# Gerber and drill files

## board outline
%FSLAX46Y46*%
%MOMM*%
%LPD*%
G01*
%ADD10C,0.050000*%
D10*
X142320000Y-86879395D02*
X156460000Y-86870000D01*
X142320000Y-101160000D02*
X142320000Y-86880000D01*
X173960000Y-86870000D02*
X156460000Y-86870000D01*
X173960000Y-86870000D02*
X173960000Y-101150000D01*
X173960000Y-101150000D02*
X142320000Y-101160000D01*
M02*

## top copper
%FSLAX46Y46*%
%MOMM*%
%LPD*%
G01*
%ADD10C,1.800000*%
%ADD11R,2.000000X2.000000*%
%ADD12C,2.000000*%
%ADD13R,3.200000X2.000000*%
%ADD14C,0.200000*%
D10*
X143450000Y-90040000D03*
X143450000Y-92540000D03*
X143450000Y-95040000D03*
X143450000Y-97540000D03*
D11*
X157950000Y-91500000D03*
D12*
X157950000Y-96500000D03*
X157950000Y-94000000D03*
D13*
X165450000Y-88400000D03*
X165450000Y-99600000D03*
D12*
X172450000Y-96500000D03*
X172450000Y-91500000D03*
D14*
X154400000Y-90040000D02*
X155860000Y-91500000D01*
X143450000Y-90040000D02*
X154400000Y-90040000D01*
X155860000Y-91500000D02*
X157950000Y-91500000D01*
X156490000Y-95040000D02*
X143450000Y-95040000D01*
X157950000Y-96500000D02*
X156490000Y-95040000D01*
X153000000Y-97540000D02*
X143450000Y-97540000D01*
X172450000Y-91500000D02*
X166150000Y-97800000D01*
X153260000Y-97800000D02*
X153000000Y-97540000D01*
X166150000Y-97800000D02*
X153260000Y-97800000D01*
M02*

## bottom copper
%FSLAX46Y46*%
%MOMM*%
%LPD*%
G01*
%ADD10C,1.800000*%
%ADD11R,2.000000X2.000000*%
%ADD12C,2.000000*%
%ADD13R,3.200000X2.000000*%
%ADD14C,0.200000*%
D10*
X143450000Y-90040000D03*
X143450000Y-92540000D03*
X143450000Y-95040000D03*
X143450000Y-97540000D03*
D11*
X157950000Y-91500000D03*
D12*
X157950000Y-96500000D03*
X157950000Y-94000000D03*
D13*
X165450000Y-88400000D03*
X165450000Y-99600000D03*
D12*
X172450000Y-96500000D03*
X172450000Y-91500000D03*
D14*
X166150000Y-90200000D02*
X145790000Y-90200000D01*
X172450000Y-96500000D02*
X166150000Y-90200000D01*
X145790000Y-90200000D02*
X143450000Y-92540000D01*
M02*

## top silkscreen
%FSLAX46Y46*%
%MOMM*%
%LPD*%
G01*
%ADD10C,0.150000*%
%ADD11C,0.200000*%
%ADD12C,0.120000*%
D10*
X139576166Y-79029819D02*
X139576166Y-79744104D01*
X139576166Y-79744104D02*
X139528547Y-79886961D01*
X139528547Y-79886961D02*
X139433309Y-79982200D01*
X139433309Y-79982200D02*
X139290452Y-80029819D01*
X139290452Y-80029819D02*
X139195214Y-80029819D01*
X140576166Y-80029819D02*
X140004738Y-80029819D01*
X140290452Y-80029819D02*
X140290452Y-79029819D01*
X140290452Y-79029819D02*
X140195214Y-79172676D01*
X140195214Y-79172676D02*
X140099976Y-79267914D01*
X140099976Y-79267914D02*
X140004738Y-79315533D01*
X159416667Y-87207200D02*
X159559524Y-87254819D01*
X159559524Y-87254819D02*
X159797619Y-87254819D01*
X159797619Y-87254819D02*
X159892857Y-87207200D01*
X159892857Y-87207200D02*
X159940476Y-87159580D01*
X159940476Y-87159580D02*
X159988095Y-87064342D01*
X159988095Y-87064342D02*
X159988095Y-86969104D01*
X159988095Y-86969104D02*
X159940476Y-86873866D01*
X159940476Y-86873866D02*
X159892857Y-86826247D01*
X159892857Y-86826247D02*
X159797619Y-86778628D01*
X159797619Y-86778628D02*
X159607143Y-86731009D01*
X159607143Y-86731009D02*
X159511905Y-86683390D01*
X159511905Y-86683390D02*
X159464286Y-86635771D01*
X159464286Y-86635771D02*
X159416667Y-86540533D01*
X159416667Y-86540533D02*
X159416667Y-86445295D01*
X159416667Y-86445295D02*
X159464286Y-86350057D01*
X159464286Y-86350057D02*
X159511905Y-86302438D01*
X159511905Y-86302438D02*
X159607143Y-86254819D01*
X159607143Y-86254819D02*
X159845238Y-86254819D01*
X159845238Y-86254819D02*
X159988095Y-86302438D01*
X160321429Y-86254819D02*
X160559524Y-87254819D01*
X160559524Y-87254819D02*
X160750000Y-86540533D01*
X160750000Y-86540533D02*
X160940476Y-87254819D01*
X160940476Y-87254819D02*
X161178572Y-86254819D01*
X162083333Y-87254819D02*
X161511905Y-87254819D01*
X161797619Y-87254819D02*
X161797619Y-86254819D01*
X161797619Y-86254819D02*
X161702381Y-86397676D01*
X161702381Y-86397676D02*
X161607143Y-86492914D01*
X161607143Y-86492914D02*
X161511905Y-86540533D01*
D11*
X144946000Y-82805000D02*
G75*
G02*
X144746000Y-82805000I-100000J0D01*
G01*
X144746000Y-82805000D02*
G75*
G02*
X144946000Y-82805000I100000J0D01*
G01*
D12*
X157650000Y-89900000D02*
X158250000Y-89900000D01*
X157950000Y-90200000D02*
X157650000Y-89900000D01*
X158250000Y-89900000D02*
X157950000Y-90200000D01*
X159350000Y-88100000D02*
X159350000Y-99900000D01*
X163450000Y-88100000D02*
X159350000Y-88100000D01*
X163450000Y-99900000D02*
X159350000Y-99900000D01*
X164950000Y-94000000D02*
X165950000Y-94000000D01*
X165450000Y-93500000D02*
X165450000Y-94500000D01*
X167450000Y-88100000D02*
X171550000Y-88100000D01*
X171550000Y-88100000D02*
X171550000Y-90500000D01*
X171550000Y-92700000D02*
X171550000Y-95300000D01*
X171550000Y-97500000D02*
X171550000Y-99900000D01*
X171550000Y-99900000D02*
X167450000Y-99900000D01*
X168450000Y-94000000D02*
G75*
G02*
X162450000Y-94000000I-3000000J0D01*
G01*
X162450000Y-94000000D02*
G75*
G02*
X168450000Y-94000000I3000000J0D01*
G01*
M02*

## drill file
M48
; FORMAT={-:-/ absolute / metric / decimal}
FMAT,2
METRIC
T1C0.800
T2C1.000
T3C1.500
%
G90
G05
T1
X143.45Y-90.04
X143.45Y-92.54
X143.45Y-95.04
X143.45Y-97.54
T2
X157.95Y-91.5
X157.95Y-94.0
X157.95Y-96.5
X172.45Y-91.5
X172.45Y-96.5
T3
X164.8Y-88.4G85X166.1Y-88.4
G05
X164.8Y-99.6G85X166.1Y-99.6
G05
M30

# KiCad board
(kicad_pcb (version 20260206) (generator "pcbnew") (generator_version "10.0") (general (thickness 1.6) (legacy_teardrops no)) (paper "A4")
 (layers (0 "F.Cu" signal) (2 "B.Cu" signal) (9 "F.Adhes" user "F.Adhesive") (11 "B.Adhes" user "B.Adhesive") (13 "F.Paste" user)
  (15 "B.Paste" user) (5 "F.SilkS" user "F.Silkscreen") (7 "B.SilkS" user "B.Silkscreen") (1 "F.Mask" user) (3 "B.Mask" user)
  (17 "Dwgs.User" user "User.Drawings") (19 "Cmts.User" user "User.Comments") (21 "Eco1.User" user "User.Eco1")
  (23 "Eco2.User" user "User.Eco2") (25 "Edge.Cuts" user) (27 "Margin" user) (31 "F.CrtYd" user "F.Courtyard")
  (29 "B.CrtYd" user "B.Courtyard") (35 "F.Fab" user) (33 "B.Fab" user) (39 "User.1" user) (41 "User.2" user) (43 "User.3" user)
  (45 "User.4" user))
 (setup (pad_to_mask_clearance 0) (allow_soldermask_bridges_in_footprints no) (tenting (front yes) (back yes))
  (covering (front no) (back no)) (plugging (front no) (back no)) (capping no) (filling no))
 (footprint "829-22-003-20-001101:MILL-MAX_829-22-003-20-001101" (layer "F.Cu") (at 140.25 82.19)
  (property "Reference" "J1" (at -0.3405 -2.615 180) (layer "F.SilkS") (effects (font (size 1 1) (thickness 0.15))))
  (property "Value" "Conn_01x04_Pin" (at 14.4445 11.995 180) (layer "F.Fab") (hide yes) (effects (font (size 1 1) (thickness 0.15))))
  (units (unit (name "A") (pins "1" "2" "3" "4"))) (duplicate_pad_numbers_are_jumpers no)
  (fp_circle (center 4.596 0.615) (end 4.596 0.715) (stroke (width 0.2) (type solid)) (fill no) (layer "F.SilkS"))
  (pad "1" thru_hole circle (at 3.2 7.85 270) (size 1.8 1.8) (drill 0.8) (layers "*.Cu" "*.Mask") (remove_unused_layers no) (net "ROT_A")
   (solder_mask_margin 0.102))
  (pad "2" thru_hole circle (at 3.2 10.35 270) (size 1.8 1.8) (drill 0.8) (layers "*.Cu" "*.Mask") (remove_unused_layers no) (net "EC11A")
   (solder_mask_margin 0.102))
  (pad "3" thru_hole circle (at 3.2 12.85 270) (size 1.8 1.8) (drill 0.8) (layers "*.Cu" "*.Mask") (remove_unused_layers no) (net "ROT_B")
   (solder_mask_margin 0.102))
  (pad "4" thru_hole circle (at 3.2 15.35 270) (size 1.8 1.8) (drill 0.8) (layers "*.Cu" "*.Mask") (remove_unused_layers no) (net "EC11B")
   (solder_mask_margin 0.102)))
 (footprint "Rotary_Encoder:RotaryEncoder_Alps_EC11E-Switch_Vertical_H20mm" (layer "F.Cu") (at 157.95 91.5)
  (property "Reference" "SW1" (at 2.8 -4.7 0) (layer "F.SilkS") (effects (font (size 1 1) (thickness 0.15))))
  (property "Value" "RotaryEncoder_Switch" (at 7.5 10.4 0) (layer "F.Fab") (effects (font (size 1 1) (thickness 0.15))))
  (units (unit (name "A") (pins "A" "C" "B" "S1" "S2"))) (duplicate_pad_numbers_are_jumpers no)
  (fp_line (start -0.3 -1.6) (end 0.3 -1.6) (stroke (width 0.12) (type solid)) (layer "F.SilkS"))
  (fp_line (start 0 -1.3) (end -0.3 -1.6) (stroke (width 0.12) (type solid)) (layer "F.SilkS"))
  (fp_line (start 0.3 -1.6) (end 0 -1.3) (stroke (width 0.12) (type solid)) (layer "F.SilkS"))
  (fp_line (start 1.4 -3.4) (end 1.4 8.4) (stroke (width 0.12) (type solid)) (layer "F.SilkS"))
  (fp_line (start 5.5 -3.4) (end 1.4 -3.4) (stroke (width 0.12) (type solid)) (layer "F.SilkS"))
  (fp_line (start 5.5 8.4) (end 1.4 8.4) (stroke (width 0.12) (type solid)) (layer "F.SilkS"))
  (fp_line (start 7 2.5) (end 8 2.5) (stroke (width 0.12) (type solid)) (layer "F.SilkS"))
  (fp_line (start 7.5 2) (end 7.5 3) (stroke (width 0.12) (type solid)) (layer "F.SilkS"))
  (fp_line (start 9.5 -3.4) (end 13.6 -3.4) (stroke (width 0.12) (type solid)) (layer "F.SilkS"))
  (fp_line (start 13.6 -3.4) (end 13.6 -1) (stroke (width 0.12) (type solid)) (layer "F.SilkS"))
  (fp_line (start 13.6 1.2) (end 13.6 3.8) (stroke (width 0.12) (type solid)) (layer "F.SilkS"))
  (fp_line (start 13.6 6) (end 13.6 8.4) (stroke (width 0.12) (type solid)) (layer "F.SilkS"))
  (fp_line (start 13.6 8.4) (end 9.5 8.4) (stroke (width 0.12) (type solid)) (layer "F.SilkS"))
  (fp_circle (center 7.5 2.5) (end 10.5 2.5) (stroke (width 0.12) (type solid)) (fill no) (layer "F.SilkS"))
  (pad "A" thru_hole rect (at 0 0) (size 2 2) (drill 1) (layers "*.Cu" "*.Mask") (remove_unused_layers no) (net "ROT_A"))
  (pad "B" thru_hole circle (at 0 5) (size 2 2) (drill 1) (layers "*.Cu" "*.Mask") (remove_unused_layers no) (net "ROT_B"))
  (pad "C" thru_hole circle (at 0 2.5) (size 2 2) (drill 1) (layers "*.Cu" "*.Mask") (remove_unused_layers no) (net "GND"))
  (pad "MP" thru_hole rect (at 7.5 -3.1) (size 3.2 2) (drill oval 2.8 1.5) (layers "*.Cu" "*.Mask") (remove_unused_layers no))
  (pad "MP" thru_hole rect (at 7.5 8.1) (size 3.2 2) (drill oval 2.8 1.5) (layers "*.Cu" "*.Mask") (remove_unused_layers no))
  (pad "S1" thru_hole circle (at 14.5 5) (size 2 2) (drill 1) (layers "*.Cu" "*.Mask") (remove_unused_layers no) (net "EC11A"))
  (pad "S2" thru_hole circle (at 14.5 0) (size 2 2) (drill 1) (layers "*.Cu" "*.Mask") (remove_unused_layers no) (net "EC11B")))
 (gr_line (start 142.32 86.879395) (end 156.46 86.87) (stroke (width 0.05) (type default)) (layer "Edge.Cuts"))
 (gr_line (start 142.32 101.16) (end 142.32 86.88) (stroke (width 0.05) (type default)) (layer "Edge.Cuts"))
 (gr_line (start 173.96 86.87) (end 156.46 86.87) (stroke (width 0.05) (type default)) (layer "Edge.Cuts"))
 (gr_line (start 173.96 86.87) (end 173.96 101.15) (stroke (width 0.05) (type default)) (layer "Edge.Cuts"))
 (gr_line (start 173.96 101.15) (end 142.32 101.16) (stroke (width 0.05) (type default)) (layer "Edge.Cuts"))
 (segment (start 154.4 90.04) (end 155.86 91.5) (width 0.2) (layer "F.Cu") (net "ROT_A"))
 (segment (start 143.45 90.04) (end 154.4 90.04) (width 0.2) (layer "F.Cu") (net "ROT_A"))
 (segment (start 155.86 91.5) (end 157.95 91.5) (width 0.2) (layer "F.Cu") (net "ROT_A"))
 (segment (start 166.15 90.2) (end 145.79 90.2) (width 0.2) (layer "B.Cu") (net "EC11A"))
 (segment (start 172.45 96.5) (end 166.15 90.2) (width 0.2) (layer "B.Cu") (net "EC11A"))
 (segment (start 145.79 90.2) (end 143.45 92.54) (width 0.2) (layer "B.Cu") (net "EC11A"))
 (segment (start 156.49 95.04) (end 143.45 95.04) (width 0.2) (layer "F.Cu") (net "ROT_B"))
 (segment (start 157.95 96.5) (end 156.49 95.04) (width 0.2) (layer "F.Cu") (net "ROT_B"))
 (segment (start 153 97.54) (end 143.45 97.54) (width 0.2) (layer "F.Cu") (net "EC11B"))
 (segment (start 172.45 91.5) (end 166.15 97.8) (width 0.2) (layer "F.Cu") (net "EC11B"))
 (segment (start 153.26 97.8) (end 153 97.54) (width 0.2) (layer "F.Cu") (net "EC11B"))
 (segment (start 166.15 97.8) (end 153.26 97.8) (width 0.2) (layer "F.Cu") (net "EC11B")))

